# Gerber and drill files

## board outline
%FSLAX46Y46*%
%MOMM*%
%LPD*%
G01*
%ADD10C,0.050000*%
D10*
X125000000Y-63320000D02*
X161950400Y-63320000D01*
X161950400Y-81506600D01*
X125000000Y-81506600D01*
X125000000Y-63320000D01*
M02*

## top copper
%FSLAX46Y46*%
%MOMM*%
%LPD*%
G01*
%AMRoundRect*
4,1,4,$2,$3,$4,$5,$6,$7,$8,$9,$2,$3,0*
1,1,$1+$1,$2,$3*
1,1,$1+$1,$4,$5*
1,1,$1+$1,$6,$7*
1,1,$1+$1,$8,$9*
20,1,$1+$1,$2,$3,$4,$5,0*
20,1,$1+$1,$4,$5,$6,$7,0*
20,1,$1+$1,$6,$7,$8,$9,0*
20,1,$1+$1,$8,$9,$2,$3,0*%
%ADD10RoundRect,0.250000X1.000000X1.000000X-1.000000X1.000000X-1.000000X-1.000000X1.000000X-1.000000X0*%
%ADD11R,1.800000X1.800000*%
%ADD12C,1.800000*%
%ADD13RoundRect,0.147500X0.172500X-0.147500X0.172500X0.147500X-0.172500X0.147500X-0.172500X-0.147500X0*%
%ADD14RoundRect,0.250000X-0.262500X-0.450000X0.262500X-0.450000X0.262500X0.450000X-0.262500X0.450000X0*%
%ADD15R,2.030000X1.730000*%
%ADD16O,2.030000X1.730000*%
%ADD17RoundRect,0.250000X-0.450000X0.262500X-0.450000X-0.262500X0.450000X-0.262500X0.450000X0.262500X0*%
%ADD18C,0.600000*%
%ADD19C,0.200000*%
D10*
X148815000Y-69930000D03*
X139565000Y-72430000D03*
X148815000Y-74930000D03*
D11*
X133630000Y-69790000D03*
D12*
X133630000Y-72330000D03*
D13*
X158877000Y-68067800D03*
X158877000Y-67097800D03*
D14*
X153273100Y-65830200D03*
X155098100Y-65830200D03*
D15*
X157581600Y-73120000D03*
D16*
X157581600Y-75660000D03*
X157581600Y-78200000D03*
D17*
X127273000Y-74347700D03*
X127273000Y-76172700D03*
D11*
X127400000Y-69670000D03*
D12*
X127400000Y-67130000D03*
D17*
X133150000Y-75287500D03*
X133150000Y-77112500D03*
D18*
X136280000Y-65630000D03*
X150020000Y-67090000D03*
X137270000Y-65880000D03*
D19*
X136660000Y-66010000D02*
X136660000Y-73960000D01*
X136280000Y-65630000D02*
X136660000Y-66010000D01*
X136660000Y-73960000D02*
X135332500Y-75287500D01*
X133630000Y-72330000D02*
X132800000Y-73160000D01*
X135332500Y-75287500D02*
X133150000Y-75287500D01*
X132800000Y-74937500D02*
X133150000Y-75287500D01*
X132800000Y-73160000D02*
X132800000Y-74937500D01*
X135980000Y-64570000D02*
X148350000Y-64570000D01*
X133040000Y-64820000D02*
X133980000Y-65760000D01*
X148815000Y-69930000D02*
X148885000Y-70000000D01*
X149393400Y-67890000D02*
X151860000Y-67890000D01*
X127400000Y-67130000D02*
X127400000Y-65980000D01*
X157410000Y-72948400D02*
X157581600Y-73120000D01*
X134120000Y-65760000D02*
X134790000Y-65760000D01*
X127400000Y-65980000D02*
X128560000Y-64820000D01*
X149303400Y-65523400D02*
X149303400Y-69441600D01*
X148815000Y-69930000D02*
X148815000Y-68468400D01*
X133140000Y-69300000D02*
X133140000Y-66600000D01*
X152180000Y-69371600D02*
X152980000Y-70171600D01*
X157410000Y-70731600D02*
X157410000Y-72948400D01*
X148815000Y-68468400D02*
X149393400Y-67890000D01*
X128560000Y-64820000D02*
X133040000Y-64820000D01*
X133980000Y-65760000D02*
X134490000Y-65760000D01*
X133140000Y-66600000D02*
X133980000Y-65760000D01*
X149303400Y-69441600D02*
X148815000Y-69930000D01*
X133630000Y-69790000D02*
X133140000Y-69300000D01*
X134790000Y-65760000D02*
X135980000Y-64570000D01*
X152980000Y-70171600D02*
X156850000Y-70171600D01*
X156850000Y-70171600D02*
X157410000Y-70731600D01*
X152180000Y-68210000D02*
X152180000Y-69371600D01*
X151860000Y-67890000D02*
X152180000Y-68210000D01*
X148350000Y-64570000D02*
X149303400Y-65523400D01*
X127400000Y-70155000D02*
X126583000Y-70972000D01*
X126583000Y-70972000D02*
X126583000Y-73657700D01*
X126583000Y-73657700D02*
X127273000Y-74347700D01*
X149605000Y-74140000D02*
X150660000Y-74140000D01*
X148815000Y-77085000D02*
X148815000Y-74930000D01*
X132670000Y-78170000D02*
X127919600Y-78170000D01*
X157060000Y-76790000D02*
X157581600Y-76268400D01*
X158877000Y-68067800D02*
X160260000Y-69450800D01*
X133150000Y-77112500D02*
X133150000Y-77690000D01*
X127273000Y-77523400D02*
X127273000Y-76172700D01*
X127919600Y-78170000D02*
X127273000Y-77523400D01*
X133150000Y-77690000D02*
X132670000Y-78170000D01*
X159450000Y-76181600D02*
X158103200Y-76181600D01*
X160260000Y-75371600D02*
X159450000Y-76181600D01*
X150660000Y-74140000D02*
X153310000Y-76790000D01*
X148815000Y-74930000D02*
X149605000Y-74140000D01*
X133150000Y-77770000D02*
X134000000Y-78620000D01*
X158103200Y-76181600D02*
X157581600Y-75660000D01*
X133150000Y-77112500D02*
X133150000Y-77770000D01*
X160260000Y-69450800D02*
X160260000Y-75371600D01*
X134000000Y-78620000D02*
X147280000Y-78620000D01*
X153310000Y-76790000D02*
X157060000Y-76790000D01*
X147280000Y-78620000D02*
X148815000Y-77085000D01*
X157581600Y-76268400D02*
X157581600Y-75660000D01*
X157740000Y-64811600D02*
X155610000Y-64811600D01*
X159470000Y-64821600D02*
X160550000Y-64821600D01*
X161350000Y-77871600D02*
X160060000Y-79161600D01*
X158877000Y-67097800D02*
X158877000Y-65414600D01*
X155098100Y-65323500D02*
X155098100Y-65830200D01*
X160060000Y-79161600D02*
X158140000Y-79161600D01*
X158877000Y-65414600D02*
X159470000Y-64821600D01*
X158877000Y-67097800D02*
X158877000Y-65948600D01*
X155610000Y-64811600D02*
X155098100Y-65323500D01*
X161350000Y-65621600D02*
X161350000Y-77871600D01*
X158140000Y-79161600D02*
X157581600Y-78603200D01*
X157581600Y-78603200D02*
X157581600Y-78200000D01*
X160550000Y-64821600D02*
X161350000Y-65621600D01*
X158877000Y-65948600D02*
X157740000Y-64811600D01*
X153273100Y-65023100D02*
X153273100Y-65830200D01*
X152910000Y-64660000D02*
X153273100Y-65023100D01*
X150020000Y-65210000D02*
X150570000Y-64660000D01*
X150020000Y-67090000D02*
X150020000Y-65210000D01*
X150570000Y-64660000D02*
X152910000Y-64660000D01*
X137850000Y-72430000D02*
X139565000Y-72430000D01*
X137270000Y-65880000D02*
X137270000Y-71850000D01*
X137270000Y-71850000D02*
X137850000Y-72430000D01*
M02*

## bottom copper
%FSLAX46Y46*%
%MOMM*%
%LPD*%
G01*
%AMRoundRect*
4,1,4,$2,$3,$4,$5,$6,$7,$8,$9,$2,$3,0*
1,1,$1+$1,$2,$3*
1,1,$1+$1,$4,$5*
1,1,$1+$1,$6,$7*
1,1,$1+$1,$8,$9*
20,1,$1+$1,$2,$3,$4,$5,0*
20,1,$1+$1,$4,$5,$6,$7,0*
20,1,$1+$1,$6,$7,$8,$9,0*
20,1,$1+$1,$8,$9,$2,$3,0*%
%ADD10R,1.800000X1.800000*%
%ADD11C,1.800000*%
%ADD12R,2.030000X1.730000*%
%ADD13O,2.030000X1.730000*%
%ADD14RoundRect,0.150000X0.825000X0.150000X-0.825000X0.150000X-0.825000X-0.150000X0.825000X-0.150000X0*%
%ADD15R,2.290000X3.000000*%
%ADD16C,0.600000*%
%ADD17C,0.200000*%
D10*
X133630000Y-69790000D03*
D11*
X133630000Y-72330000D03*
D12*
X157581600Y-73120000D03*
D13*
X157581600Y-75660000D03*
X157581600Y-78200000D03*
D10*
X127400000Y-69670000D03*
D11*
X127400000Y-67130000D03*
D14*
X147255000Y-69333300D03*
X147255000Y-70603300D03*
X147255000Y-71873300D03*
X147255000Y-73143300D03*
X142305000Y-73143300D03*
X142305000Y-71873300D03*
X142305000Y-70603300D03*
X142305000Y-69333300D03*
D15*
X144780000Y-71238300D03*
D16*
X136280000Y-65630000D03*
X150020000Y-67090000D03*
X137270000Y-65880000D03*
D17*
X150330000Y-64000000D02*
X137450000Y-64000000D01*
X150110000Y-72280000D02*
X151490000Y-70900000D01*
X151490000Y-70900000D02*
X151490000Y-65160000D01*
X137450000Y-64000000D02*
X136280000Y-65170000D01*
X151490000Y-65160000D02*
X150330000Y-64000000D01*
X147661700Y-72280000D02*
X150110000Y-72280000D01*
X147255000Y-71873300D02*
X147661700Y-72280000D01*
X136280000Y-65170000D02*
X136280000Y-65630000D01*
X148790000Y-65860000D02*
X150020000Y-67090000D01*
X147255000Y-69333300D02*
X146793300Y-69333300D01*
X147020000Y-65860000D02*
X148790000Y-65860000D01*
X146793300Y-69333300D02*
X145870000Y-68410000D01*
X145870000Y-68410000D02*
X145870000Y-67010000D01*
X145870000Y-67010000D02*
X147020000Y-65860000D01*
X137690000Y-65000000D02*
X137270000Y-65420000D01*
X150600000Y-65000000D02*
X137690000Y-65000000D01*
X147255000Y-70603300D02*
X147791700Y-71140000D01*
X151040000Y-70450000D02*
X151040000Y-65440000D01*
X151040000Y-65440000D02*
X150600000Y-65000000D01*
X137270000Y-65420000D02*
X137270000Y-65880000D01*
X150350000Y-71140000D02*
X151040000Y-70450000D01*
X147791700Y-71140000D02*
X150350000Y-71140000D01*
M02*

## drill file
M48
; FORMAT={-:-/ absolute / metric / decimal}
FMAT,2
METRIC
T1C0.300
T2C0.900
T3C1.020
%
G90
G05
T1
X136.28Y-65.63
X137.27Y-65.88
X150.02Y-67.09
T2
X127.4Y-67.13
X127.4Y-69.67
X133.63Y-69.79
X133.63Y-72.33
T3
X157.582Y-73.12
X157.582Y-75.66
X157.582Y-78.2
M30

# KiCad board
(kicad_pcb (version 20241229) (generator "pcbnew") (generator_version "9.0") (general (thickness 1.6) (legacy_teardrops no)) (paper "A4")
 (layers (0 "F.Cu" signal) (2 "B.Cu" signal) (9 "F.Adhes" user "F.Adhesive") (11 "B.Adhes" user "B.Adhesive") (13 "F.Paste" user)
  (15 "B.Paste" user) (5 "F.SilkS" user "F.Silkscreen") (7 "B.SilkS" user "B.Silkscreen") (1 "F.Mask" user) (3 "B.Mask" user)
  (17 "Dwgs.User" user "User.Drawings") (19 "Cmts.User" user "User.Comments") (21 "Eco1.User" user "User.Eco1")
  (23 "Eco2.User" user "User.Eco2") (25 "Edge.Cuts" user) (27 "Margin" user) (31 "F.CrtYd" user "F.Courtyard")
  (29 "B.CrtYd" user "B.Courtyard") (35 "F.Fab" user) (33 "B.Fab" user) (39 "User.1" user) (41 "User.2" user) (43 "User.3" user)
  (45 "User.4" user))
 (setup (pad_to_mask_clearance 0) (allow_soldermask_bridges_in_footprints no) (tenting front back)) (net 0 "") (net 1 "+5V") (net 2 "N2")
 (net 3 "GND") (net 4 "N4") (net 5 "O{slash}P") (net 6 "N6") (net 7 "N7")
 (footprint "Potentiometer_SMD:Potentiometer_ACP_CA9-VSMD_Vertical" (layer "F.Cu") (at 144.19 72.43 180)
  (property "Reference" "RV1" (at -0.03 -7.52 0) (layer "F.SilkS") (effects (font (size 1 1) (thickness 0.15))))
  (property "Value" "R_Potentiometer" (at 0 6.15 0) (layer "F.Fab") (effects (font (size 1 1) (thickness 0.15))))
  (pad "1" smd roundrect (at -4.625 2.5 180) (size 2.5 2.5) (layers "F.Cu" "F.Mask" "F.Paste") (roundrect_rratio 0.1) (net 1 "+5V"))
  (pad "2" smd roundrect (at 4.625 0 180) (size 2.5 2.5) (layers "F.Cu" "F.Mask" "F.Paste") (roundrect_rratio 0.1) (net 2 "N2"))
  (pad "3" smd roundrect (at -4.625 -2.5 180) (size 2.5 2.5) (layers "F.Cu" "F.Mask" "F.Paste") (roundrect_rratio 0.1) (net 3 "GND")))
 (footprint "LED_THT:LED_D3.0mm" (layer "F.Cu") (at 133.63 69.79 -90)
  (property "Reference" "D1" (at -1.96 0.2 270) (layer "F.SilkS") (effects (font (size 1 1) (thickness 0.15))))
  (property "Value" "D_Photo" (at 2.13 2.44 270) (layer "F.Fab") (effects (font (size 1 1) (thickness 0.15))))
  (pad "1" thru_hole rect (at 0 0 270) (size 1.8 1.8) (drill 0.9) (layers "*.Cu" "*.Mask") (remove_unused_layers no) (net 1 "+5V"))
  (pad "2" thru_hole circle (at 2.54 0 270) (size 1.8 1.8) (drill 0.9) (layers "*.Cu" "*.Mask") (remove_unused_layers no) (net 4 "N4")))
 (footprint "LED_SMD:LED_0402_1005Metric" (layer "F.Cu") (at 158.877 67.5828 90)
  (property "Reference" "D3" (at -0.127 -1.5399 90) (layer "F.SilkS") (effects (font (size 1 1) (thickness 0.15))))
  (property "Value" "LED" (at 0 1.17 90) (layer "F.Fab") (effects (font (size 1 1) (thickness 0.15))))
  (pad "1" smd roundrect (at -0.485 0 90) (size 0.59 0.64) (layers "F.Cu" "F.Mask" "F.Paste") (roundrect_rratio 0.25) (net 3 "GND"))
  (pad "2" smd roundrect (at 0.485 0 90) (size 0.59 0.64) (layers "F.Cu" "F.Mask" "F.Paste") (roundrect_rratio 0.25) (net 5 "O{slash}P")))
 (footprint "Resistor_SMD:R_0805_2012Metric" (layer "F.Cu") (at 154.1856 65.8302)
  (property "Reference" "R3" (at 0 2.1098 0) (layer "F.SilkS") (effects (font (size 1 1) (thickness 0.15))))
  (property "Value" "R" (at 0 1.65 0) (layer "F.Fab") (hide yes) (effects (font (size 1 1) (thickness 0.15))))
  (pad "1" smd roundrect (at -0.9125 0) (size 1.025 1.4) (layers "F.Cu" "F.Mask" "F.Paste") (roundrect_rratio 0.243902) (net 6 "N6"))
  (pad "2" smd roundrect (at 0.9125 0) (size 1.025 1.4) (layers "F.Cu" "F.Mask" "F.Paste") (roundrect_rratio 0.243902) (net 5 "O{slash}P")))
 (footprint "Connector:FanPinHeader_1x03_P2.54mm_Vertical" (layer "F.Cu") (at 157.5816 73.12 -90)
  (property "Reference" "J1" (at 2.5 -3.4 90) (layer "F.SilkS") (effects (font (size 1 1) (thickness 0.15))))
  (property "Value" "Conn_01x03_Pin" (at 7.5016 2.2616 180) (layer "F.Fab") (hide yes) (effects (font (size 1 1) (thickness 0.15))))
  (pad "1" thru_hole rect (at 0 0) (size 2.03 1.73) (drill 1.02) (layers "*.Cu" "*.Mask") (remove_unused_layers no) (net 1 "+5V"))
  (pad "2" thru_hole oval (at 2.54 0) (size 2.03 1.73) (drill 1.02) (layers "*.Cu" "*.Mask") (remove_unused_layers no) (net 3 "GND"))
  (pad "3" thru_hole oval (at 5.08 0) (size 2.03 1.73) (drill 1.02) (layers "*.Cu" "*.Mask") (remove_unused_layers no) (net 5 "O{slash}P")))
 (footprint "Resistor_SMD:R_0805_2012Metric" (layer "F.Cu") (at 127.273 75.2602 -90)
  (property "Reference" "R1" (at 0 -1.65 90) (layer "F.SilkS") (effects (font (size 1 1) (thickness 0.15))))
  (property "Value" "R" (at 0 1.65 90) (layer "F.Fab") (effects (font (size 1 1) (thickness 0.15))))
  (pad "1" smd roundrect (at -0.9125 0 270) (size 1.025 1.4) (layers "F.Cu" "F.Mask" "F.Paste") (roundrect_rratio 0.243902) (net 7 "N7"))
  (pad "2" smd roundrect (at 0.9125 0 270) (size 1.025 1.4) (layers "F.Cu" "F.Mask" "F.Paste") (roundrect_rratio 0.243902) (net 3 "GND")))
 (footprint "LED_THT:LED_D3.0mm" (layer "F.Cu") (at 127.4 69.67 90)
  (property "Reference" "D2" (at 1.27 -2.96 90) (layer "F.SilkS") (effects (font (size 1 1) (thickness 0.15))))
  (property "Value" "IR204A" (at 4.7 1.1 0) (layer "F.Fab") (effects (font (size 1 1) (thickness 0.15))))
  (pad "1" thru_hole rect (at 0 0 90) (size 1.8 1.8) (drill 0.9) (layers "*.Cu" "*.Mask") (remove_unused_layers no) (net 7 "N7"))
  (pad "2" thru_hole circle (at 2.54 0 90) (size 1.8 1.8) (drill 0.9) (layers "*.Cu" "*.Mask") (remove_unused_layers no) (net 1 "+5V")))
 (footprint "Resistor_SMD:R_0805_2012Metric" (layer "F.Cu") (at 133.15 76.2 -90)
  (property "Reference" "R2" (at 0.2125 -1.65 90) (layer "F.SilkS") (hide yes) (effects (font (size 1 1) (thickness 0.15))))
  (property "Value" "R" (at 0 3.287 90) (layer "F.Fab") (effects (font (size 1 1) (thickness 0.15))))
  (pad "1" smd roundrect (at -0.9125 0 270) (size 1.025 1.4) (layers "F.Cu" "F.Mask" "F.Paste") (roundrect_rratio 0.243902) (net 4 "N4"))
  (pad "2" smd roundrect (at 0.9125 0 270) (size 1.025 1.4) (layers "F.Cu" "F.Mask" "F.Paste") (roundrect_rratio 0.243902) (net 3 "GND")))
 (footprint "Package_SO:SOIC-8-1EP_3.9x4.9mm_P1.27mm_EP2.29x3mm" (layer "B.Cu") (at 144.78 71.2383 180)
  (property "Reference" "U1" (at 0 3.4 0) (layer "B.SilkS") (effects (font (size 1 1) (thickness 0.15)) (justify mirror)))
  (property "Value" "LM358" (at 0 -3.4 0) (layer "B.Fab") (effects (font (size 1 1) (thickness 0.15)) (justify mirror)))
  (pad "" smd roundrect (at -0.57 -0.75 180) (size 0.92 1.21) (layers "B.Paste") (roundrect_rratio 0.25))
  (pad "" smd roundrect (at -0.57 0.75 180) (size 0.92 1.21) (layers "B.Paste") (roundrect_rratio 0.25))
  (pad "" smd roundrect (at 0.57 -0.75 180) (size 0.92 1.21) (layers "B.Paste") (roundrect_rratio 0.25))
  (pad "" smd roundrect (at 0.57 0.75 180) (size 0.92 1.21) (layers "B.Paste") (roundrect_rratio 0.25))
  (pad "1" smd roundrect (at -2.475 1.905 180) (size 1.95 0.6) (layers "B.Cu" "B.Mask" "B.Paste") (roundrect_rratio 0.25) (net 6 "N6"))
  (pad "2" smd roundrect (at -2.475 0.635 180) (size 1.95 0.6) (layers "B.Cu" "B.Mask" "B.Paste") (roundrect_rratio 0.25) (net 2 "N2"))
  (pad "3" smd roundrect (at -2.475 -0.635 180) (size 1.95 0.6) (layers "B.Cu" "B.Mask" "B.Paste") (roundrect_rratio 0.25) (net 4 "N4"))
  (pad "4" smd roundrect (at -2.475 -1.905 180) (size 1.95 0.6) (layers "B.Cu" "B.Mask" "B.Paste") (roundrect_rratio 0.25))
  (pad "5" smd roundrect (at 2.475 -1.905 180) (size 1.95 0.6) (layers "B.Cu" "B.Mask" "B.Paste") (roundrect_rratio 0.25))
  (pad "6" smd roundrect (at 2.475 -0.635 180) (size 1.95 0.6) (layers "B.Cu" "B.Mask" "B.Paste") (roundrect_rratio 0.25))
  (pad "7" smd roundrect (at 2.475 0.635 180) (size 1.95 0.6) (layers "B.Cu" "B.Mask" "B.Paste") (roundrect_rratio 0.25))
  (pad "8" smd roundrect (at 2.475 1.905 180) (size 1.95 0.6) (layers "B.Cu" "B.Mask" "B.Paste") (roundrect_rratio 0.25))
  (pad "9" smd rect (at 0 0 180) (size 2.29 3) (layers "B.Cu" "B.Mask") (zone_connect 2)))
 (gr_rect (start 125 63.32) (end 161.9504 81.5066) (stroke (width 0.05) (type default)) (fill no) (layer "Edge.Cuts"))
 (segment (start 136.66 66.01) (end 136.66 73.96) (width 0.2) (layer "F.Cu") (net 4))
 (segment (start 136.28 65.63) (end 136.66 66.01) (width 0.2) (layer "F.Cu") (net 4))
 (segment (start 136.66 73.96) (end 135.3325 75.2875) (width 0.2) (layer "F.Cu") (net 4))
 (segment (start 133.63 72.33) (end 132.8 73.16) (width 0.2) (layer "F.Cu") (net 4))
 (segment (start 135.3325 75.2875) (end 133.15 75.2875) (width 0.2) (layer "F.Cu") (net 4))
 (segment (start 132.8 74.9375) (end 133.15 75.2875) (width 0.2) (layer "F.Cu") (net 4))
 (segment (start 132.8 73.16) (end 132.8 74.9375) (width 0.2) (layer "F.Cu") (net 4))
 (via (at 136.28 65.63) (size 0.6) (drill 0.3) (layers "F.Cu" "B.Cu") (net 4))
 (segment (start 150.33 64) (end 137.45 64) (width 0.2) (layer "B.Cu") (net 4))
 (segment (start 150.11 72.28) (end 151.49 70.9) (width 0.2) (layer "B.Cu") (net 4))
 (segment (start 151.49 70.9) (end 151.49 65.16) (width 0.2) (layer "B.Cu") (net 4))
 (segment (start 137.45 64) (end 136.28 65.17) (width 0.2) (layer "B.Cu") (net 4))
 (segment (start 151.49 65.16) (end 150.33 64) (width 0.2) (layer "B.Cu") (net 4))
 (segment (start 147.6617 72.28) (end 150.11 72.28) (width 0.2) (layer "B.Cu") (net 4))
 (segment (start 147.255 71.8733) (end 147.6617 72.28) (width 0.2) (layer "B.Cu") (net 4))
 (segment (start 136.28 65.17) (end 136.28 65.63) (width 0.2) (layer "B.Cu") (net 4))
 (segment (start 135.98 64.57) (end 148.35 64.57) (width 0.2) (layer "F.Cu") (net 1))
 (segment (start 133.04 64.82) (end 133.98 65.76) (width 0.2) (layer "F.Cu") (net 1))
 (segment (start 148.815 69.93) (end 148.885 70) (width 0.2) (layer "F.Cu") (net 1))
 (segment (start 149.3934 67.89) (end 151.86 67.89) (width 0.2) (layer "F.Cu") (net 1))
 (segment (start 127.4 67.13) (end 127.4 65.98) (width 0.2) (layer "F.Cu") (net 1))
 (segment (start 157.41 72.9484) (end 157.5816 73.12) (width 0.2) (layer "F.Cu") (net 1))
 (segment (start 134.12 65.76) (end 134.79 65.76) (width 0.2) (layer "F.Cu") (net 1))
 (segment (start 127.4 65.98) (end 128.56 64.82) (width 0.2) (layer "F.Cu") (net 1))
 (segment (start 149.3034 65.5234) (end 149.3034 69.4416) (width 0.2) (layer "F.Cu") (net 1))
 (segment (start 148.815 69.93) (end 148.815 68.4684) (width 0.2) (layer "F.Cu") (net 1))
 (segment (start 133.14 69.3) (end 133.14 66.6) (width 0.2) (layer "F.Cu") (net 1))
 (segment (start 152.18 69.3716) (end 152.98 70.1716) (width 0.2) (layer "F.Cu") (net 1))
 (segment (start 157.41 70.7316) (end 157.41 72.9484) (width 0.2) (layer "F.Cu") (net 1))
 (segment (start 148.815 68.4684) (end 149.3934 67.89) (width 0.2) (layer "F.Cu") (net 1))
 (segment (start 128.56 64.82) (end 133.04 64.82) (width 0.2) (layer "F.Cu") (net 1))
 (segment (start 133.98 65.76) (end 134.49 65.76) (width 0.2) (layer "F.Cu") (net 1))
 (segment (start 133.14 66.6) (end 133.98 65.76) (width 0.2) (layer "F.Cu") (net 1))
 (segment (start 149.3034 69.4416) (end 148.815 69.93) (width 0.2) (layer "F.Cu") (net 1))
 (segment (start 133.63 69.79) (end 133.14 69.3) (width 0.2) (layer "F.Cu") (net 1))
 (segment (start 134.79 65.76) (end 135.98 64.57) (width 0.2) (layer "F.Cu") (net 1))
 (segment (start 152.98 70.1716) (end 156.85 70.1716) (width 0.2) (layer "F.Cu") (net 1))
 (segment (start 156.85 70.1716) (end 157.41 70.7316) (width 0.2) (layer "F.Cu") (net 1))
 (segment (start 152.18 68.21) (end 152.18 69.3716) (width 0.2) (layer "F.Cu") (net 1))
 (segment (start 151.86 67.89) (end 152.18 68.21) (width 0.2) (layer "F.Cu") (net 1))
 (segment (start 148.35 64.57) (end 149.3034 65.5234) (width 0.2) (layer "F.Cu") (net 1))
 (segment (start 127.4 70.155) (end 126.583 70.972) (width 0.2) (layer "F.Cu") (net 7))
 (segment (start 126.583 70.972) (end 126.583 73.6577) (width 0.2) (layer "F.Cu") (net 7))
 (segment (start 126.583 73.6577) (end 127.273 74.3477) (width 0.2) (layer "F.Cu") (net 7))
 (segment (start 149.605 74.14) (end 150.66 74.14) (width 0.2) (layer "F.Cu") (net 3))
 (segment (start 148.815 77.085) (end 148.815 74.93) (width 0.2) (layer "F.Cu") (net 3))
 (segment (start 132.67 78.17) (end 127.9196 78.17) (width 0.2) (layer "F.Cu") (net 3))
 (segment (start 157.06 76.79) (end 157.5816 76.2684) (width 0.2) (layer "F.Cu") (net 3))
 (segment (start 158.877 68.0678) (end 160.26 69.4508) (width 0.2) (layer "F.Cu") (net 3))
 (segment (start 133.15 77.1125) (end 133.15 77.69) (width 0.2) (layer "F.Cu") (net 3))
 (segment (start 127.273 77.5234) (end 127.273 76.1727) (width 0.2) (layer "F.Cu") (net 3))
 (segment (start 127.9196 78.17) (end 127.273 77.5234) (width 0.2) (layer "F.Cu") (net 3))
 (segment (start 133.15 77.69) (end 132.67 78.17) (width 0.2) (layer "F.Cu") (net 3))
 (segment (start 159.45 76.1816) (end 158.1032 76.1816) (width 0.2) (layer "F.Cu") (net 3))
 (segment (start 160.26 75.3716) (end 159.45 76.1816) (width 0.2) (layer "F.Cu") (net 3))
 (segment (start 150.66 74.14) (end 153.31 76.79) (width 0.2) (layer "F.Cu") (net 3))
 (segment (start 148.815 74.93) (end 149.605 74.14) (width 0.2) (layer "F.Cu") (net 3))
 (segment (start 133.15 77.77) (end 134 78.62) (width 0.2) (layer "F.Cu") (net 3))
 (segment (start 158.1032 76.1816) (end 157.5816 75.66) (width 0.2) (layer "F.Cu") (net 3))
 (segment (start 133.15 77.1125) (end 133.15 77.77) (width 0.2) (layer "F.Cu") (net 3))
 (segment (start 160.26 69.4508) (end 160.26 75.3716) (width 0.2) (layer "F.Cu") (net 3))
 (segment (start 134 78.62) (end 147.28 78.62) (width 0.2) (layer "F.Cu") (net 3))
 (segment (start 153.31 76.79) (end 157.06 76.79) (width 0.2) (layer "F.Cu") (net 3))
 (segment (start 147.28 78.62) (end 148.815 77.085) (width 0.2) (layer "F.Cu") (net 3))
 (segment (start 157.5816 76.2684) (end 157.5816 75.66) (width 0.2) (layer "F.Cu") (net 3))
 (segment (start 157.74 64.8116) (end 155.61 64.8116) (width 0.2) (layer "F.Cu") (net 5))
 (segment (start 159.47 64.8216) (end 160.55 64.8216) (width 0.2) (layer "F.Cu") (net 5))
 (segment (start 161.35 77.8716) (end 160.06 79.1616) (width 0.2) (layer "F.Cu") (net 5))
 (segment (start 158.877 67.0978) (end 158.877 65.4146) (width 0.2) (layer "F.Cu") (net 5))
 (segment (start 155.0981 65.3235) (end 155.0981 65.8302) (width 0.2) (layer "F.Cu") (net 5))
 (segment (start 160.06 79.1616) (end 158.14 79.1616) (width 0.2) (layer "F.Cu") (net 5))
 (segment (start 158.877 65.4146) (end 159.47 64.8216) (width 0.2) (layer "F.Cu") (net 5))
 (segment (start 158.877 67.0978) (end 158.877 65.9486) (width 0.2) (layer "F.Cu") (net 5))
 (segment (start 155.61 64.8116) (end 155.0981 65.3235) (width 0.2) (layer "F.Cu") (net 5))
 (segment (start 161.35 65.6216) (end 161.35 77.8716) (width 0.2) (layer "F.Cu") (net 5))
 (segment (start 158.14 79.1616) (end 157.5816 78.6032) (width 0.2) (layer "F.Cu") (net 5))
 (segment (start 157.5816 78.6032) (end 157.5816 78.2) (width 0.2) (layer "F.Cu") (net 5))
 (segment (start 160.55 64.8216) (end 161.35 65.6216) (width 0.2) (layer "F.Cu") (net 5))
 (segment (start 158.877 65.9486) (end 157.74 64.8116) (width 0.2) (layer "F.Cu") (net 5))
 (segment (start 153.2731 65.0231) (end 153.2731 65.8302) (width 0.2) (layer "F.Cu") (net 6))
 (segment (start 152.91 64.66) (end 153.2731 65.0231) (width 0.2) (layer "F.Cu") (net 6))
 (segment (start 150.02 65.21) (end 150.57 64.66) (width 0.2) (layer "F.Cu") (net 6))
 (segment (start 150.02 67.09) (end 150.02 65.21) (width 0.2) (layer "F.Cu") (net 6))
 (segment (start 150.57 64.66) (end 152.91 64.66) (width 0.2) (layer "F.Cu") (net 6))
 (via (at 150.02 67.09) (size 0.6) (drill 0.3) (layers "F.Cu" "B.Cu") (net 6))
 (segment (start 148.79 65.86) (end 150.02 67.09) (width 0.2) (layer "B.Cu") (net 6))
 (segment (start 147.255 69.3333) (end 146.7933 69.3333) (width 0.2) (layer "B.Cu") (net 6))
 (segment (start 147.02 65.86) (end 148.79 65.86) (width 0.2) (layer "B.Cu") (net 6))
 (segment (start 146.7933 69.3333) (end 145.87 68.41) (width 0.2) (layer "B.Cu") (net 6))
 (segment (start 145.87 68.41) (end 145.87 67.01) (width 0.2) (layer "B.Cu") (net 6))
 (segment (start 145.87 67.01) (end 147.02 65.86) (width 0.2) (layer "B.Cu") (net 6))
 (segment (start 137.85 72.43) (end 139.565 72.43) (width 0.2) (layer "F.Cu") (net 2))
 (segment (start 137.27 65.88) (end 137.27 71.85) (width 0.2) (layer "F.Cu") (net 2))
 (segment (start 137.27 71.85) (end 137.85 72.43) (width 0.2) (layer "F.Cu") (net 2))
 (via (at 137.27 65.88) (size 0.6) (drill 0.3) (layers "F.Cu" "B.Cu") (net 2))
 (segment (start 137.69 65) (end 137.27 65.42) (width 0.2) (layer "B.Cu") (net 2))
 (segment (start 150.6 65) (end 137.69 65) (width 0.2) (layer "B.Cu") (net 2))
 (segment (start 147.255 70.6033) (end 147.7917 71.14) (width 0.2) (layer "B.Cu") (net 2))
 (segment (start 151.04 70.45) (end 151.04 65.44) (width 0.2) (layer "B.Cu") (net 2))
 (segment (start 151.04 65.44) (end 150.6 65) (width 0.2) (layer "B.Cu") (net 2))
 (segment (start 137.27 65.42) (end 137.27 65.88) (width 0.2) (layer "B.Cu") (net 2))
 (segment (start 150.35 71.14) (end 151.04 70.45) (width 0.2) (layer "B.Cu") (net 2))
 (segment (start 147.7917 71.14) (end 150.35 71.14) (width 0.2) (layer "B.Cu") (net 2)))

